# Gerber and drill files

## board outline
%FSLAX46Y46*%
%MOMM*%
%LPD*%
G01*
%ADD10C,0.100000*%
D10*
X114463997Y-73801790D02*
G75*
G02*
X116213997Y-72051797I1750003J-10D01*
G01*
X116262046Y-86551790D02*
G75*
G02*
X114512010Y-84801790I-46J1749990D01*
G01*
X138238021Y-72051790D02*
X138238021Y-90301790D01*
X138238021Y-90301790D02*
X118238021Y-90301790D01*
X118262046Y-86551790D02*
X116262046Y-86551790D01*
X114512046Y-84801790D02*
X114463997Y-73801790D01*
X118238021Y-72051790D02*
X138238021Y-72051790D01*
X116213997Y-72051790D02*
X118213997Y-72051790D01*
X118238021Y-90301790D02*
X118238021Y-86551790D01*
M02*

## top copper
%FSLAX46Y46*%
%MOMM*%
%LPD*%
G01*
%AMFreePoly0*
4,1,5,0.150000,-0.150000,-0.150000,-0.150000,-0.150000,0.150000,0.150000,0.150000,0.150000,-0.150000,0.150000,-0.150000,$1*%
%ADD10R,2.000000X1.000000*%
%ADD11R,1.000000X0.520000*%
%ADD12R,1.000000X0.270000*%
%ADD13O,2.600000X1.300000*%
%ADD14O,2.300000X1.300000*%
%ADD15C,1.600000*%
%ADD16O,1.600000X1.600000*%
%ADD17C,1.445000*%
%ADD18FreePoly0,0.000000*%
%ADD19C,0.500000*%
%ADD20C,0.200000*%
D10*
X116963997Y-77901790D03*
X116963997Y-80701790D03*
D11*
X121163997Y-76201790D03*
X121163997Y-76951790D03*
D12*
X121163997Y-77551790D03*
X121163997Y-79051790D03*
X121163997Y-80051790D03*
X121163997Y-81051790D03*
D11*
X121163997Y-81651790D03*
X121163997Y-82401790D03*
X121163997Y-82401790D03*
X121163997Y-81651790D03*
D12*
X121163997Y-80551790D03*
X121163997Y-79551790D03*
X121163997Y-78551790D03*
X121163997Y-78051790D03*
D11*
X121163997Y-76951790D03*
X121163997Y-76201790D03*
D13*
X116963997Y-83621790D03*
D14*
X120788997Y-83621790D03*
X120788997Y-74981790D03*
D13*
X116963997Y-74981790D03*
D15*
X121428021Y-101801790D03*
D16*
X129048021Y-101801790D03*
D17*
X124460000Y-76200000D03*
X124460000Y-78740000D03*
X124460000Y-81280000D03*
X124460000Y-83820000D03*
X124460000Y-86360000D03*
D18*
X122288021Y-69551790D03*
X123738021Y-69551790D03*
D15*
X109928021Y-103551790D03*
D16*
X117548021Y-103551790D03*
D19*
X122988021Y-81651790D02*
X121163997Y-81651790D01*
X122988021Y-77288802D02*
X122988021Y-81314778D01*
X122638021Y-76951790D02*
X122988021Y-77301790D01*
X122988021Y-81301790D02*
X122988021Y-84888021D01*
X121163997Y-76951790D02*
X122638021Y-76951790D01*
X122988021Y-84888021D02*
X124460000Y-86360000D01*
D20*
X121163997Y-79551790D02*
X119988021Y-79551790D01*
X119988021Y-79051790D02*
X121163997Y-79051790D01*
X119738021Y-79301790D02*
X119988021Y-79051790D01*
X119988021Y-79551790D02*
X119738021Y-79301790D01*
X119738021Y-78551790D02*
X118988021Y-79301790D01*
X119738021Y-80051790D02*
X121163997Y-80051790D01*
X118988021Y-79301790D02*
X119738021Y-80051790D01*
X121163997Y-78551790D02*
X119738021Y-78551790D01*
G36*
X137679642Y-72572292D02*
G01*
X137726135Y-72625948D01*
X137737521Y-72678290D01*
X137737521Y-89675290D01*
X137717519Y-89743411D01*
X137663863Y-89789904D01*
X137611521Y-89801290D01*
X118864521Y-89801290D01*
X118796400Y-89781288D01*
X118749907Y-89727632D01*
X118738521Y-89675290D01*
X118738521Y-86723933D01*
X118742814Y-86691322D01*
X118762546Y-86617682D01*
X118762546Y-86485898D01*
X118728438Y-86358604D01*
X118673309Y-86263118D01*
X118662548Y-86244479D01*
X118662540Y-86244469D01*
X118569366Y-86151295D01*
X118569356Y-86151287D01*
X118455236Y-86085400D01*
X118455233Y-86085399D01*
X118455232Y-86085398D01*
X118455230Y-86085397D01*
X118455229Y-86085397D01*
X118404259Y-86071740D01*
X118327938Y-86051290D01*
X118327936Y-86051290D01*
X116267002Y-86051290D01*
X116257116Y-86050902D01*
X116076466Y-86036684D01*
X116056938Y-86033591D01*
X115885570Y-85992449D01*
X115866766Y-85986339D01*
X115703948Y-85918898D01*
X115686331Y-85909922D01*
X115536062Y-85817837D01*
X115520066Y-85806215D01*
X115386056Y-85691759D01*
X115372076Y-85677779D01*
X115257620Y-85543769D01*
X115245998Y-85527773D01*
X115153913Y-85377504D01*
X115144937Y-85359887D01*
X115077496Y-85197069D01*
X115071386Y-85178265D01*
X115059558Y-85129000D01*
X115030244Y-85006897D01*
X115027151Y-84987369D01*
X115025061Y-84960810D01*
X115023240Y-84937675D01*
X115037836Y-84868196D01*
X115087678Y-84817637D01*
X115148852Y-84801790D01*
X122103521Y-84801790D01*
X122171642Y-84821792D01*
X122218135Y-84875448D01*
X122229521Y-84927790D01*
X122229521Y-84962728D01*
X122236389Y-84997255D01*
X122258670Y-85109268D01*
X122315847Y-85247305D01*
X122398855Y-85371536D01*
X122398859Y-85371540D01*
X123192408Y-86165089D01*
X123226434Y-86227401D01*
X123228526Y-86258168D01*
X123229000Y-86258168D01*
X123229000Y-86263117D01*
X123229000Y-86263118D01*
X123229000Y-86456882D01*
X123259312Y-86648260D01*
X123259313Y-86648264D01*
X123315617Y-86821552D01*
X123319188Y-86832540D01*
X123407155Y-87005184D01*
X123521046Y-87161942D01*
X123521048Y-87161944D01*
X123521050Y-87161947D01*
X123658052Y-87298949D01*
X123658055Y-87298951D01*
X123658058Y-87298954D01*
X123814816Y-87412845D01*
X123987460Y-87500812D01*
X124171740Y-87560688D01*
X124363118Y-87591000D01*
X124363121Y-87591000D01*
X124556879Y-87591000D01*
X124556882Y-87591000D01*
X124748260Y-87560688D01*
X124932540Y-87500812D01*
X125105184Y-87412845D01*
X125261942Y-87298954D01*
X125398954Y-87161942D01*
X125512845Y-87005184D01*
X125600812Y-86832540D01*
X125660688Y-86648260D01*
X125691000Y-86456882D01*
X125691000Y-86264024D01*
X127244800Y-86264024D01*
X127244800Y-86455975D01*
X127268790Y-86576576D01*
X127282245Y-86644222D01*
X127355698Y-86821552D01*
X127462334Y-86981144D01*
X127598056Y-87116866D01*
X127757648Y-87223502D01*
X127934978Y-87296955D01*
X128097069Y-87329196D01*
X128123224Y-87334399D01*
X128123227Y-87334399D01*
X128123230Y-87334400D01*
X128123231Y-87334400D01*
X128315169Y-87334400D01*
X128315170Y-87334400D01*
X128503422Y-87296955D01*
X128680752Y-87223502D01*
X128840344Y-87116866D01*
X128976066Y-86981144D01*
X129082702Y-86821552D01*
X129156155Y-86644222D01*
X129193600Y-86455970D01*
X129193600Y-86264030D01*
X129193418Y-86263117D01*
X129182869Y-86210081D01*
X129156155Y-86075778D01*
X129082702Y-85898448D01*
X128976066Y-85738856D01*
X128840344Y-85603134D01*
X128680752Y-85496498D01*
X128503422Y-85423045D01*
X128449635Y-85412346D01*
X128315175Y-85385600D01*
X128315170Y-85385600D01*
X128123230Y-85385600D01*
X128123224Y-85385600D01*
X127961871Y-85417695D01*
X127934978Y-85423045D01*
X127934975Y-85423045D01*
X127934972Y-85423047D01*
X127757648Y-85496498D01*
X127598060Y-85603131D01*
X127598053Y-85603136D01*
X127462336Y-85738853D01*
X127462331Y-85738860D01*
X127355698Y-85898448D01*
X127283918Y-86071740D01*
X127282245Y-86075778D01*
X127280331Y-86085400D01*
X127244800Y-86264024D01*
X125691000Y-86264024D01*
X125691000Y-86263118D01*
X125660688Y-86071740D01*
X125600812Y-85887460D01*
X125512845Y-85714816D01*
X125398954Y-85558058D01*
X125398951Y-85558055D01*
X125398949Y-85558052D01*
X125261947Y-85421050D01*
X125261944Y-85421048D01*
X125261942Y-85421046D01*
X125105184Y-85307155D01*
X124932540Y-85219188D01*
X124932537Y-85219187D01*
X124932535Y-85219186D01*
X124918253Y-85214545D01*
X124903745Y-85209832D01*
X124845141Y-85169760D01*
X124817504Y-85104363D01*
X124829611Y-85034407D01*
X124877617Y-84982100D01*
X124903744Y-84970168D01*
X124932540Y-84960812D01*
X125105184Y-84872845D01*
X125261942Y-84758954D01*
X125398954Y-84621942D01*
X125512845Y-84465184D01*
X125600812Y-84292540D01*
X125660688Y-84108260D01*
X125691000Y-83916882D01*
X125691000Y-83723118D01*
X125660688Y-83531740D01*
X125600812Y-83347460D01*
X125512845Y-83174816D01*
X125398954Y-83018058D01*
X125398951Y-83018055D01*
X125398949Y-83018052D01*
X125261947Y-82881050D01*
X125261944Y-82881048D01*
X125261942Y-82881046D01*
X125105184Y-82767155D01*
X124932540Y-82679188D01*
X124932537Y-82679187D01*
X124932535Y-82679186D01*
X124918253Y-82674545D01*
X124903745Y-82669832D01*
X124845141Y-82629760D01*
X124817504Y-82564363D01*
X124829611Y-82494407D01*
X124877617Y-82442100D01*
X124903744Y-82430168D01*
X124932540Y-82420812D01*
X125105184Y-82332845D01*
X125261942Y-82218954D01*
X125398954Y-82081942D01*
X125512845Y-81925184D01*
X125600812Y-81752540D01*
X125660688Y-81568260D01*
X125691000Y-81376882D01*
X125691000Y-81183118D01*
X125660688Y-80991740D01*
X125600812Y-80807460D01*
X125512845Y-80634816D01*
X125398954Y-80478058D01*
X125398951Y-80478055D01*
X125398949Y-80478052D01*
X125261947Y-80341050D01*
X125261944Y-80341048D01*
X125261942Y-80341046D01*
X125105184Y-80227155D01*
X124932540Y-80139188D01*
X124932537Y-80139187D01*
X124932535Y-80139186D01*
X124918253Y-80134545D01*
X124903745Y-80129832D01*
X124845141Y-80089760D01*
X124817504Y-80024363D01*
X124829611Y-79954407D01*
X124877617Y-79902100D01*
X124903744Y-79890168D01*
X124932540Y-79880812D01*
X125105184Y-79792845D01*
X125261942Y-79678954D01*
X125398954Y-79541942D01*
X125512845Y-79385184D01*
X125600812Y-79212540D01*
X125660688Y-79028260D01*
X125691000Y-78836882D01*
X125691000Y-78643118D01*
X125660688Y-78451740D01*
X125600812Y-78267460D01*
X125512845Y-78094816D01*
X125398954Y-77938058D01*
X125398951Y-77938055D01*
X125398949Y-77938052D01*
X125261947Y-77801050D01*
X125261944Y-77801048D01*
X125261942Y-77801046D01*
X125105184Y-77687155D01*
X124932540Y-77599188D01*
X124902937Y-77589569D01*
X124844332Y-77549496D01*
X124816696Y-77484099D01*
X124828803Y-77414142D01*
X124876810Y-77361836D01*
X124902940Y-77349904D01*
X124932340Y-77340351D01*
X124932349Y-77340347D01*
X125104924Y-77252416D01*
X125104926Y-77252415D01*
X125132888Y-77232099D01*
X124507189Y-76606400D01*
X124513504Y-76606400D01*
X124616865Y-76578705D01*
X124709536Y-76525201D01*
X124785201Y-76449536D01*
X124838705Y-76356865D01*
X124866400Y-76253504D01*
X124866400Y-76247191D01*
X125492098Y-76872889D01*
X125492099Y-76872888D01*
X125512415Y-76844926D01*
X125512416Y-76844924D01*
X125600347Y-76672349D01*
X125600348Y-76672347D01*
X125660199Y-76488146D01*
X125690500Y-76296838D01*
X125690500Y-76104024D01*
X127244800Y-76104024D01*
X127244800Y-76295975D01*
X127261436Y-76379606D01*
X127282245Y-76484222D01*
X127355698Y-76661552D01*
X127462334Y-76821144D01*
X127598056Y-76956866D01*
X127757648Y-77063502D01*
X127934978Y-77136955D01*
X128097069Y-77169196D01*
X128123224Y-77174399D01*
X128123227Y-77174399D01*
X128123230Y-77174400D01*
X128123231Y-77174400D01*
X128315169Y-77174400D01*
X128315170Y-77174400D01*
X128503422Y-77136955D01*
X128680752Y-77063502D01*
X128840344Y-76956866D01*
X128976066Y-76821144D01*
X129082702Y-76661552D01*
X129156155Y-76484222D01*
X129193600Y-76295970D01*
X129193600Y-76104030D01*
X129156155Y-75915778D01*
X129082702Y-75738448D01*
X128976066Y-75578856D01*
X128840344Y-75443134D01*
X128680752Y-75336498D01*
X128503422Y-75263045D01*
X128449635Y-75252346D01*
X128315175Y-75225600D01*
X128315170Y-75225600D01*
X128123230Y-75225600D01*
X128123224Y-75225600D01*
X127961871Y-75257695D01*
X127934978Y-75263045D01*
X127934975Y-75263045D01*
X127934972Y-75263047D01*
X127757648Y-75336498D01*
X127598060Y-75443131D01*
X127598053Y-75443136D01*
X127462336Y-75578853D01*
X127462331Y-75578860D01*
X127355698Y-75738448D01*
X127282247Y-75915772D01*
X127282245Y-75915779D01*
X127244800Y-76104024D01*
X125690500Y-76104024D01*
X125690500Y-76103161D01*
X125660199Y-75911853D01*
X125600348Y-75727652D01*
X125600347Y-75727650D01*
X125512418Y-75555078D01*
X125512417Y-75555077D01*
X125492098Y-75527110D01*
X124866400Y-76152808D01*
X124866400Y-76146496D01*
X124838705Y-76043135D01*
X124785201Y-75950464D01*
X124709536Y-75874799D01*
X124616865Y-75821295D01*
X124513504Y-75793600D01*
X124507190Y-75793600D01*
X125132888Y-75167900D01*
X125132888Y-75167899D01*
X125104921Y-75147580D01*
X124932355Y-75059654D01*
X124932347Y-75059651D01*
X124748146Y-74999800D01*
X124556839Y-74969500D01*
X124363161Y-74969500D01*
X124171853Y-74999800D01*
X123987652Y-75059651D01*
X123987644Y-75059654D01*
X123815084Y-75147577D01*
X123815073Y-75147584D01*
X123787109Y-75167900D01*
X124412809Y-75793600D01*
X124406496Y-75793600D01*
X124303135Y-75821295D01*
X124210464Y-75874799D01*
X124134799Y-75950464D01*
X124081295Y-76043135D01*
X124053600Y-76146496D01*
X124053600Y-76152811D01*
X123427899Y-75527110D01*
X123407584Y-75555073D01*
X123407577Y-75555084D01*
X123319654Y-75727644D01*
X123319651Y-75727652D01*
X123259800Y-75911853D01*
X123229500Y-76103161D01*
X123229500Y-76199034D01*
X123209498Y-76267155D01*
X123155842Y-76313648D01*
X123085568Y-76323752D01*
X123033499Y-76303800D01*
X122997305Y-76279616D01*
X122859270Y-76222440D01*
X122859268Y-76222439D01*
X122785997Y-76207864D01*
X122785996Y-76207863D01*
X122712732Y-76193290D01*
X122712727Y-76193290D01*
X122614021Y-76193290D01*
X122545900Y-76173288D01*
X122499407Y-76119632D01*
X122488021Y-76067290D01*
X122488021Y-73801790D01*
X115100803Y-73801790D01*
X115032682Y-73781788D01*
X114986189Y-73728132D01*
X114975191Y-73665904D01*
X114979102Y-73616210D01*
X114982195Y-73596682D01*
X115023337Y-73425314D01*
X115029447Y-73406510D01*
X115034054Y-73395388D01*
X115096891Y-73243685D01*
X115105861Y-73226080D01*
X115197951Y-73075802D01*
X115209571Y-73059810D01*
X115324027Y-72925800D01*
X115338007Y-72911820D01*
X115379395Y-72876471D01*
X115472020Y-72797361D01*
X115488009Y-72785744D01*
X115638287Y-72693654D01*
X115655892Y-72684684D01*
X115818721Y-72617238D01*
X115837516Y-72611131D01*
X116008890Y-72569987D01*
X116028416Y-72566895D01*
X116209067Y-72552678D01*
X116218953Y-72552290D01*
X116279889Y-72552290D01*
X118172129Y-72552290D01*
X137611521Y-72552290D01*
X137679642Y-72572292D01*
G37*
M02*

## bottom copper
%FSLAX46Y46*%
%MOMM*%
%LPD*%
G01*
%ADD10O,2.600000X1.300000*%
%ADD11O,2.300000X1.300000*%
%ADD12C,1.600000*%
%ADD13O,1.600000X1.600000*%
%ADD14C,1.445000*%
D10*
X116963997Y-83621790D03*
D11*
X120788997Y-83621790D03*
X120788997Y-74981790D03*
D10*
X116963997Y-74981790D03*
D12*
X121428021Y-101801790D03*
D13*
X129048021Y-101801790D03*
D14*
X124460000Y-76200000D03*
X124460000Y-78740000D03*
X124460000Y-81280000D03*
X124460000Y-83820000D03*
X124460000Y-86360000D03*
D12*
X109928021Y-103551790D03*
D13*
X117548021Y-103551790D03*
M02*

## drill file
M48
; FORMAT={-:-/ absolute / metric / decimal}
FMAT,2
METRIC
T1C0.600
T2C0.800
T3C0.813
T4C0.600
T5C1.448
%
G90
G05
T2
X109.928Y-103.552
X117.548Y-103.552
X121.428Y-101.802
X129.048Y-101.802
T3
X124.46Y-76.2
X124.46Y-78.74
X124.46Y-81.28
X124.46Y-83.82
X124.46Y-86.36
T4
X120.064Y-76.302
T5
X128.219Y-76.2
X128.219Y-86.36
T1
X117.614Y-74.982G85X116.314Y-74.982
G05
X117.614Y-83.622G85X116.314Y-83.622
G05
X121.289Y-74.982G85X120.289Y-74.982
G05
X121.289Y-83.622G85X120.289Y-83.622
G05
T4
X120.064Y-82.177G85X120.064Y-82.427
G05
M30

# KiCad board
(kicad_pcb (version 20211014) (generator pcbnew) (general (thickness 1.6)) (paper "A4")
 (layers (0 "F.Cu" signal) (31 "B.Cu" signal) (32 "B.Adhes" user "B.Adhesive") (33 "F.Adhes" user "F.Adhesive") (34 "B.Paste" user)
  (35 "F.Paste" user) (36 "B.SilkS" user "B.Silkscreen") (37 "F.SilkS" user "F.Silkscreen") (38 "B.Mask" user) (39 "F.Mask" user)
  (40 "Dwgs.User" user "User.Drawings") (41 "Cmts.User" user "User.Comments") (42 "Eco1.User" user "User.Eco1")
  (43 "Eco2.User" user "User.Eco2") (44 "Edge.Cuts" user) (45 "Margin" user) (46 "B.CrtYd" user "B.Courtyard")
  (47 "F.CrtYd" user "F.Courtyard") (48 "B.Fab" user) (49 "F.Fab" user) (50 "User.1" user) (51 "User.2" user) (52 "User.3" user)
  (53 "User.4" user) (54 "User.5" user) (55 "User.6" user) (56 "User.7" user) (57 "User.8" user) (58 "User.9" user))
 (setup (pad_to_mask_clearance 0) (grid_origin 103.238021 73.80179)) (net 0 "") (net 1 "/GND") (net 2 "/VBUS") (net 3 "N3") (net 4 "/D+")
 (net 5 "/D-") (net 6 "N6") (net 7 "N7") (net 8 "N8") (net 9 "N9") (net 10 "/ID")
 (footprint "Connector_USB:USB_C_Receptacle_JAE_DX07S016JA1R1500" (layer "F.Cu") (at 118.113997 79.30179 -90)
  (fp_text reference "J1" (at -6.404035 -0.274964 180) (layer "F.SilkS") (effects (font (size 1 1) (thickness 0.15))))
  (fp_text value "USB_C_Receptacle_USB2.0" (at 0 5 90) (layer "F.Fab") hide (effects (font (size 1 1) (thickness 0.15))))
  (pad "" smd rect (at -1.4 1.15 270) (size 1 2) (layers "F.Cu" "F.Paste" "F.Mask"))
  (pad "" np_thru_hole circle (at -3 -1.95 270) (size 0.6 0.6) (drill 0.6) (layers F&B.Cu *.Mask))
  (pad "" np_thru_hole oval (at 3 -1.95 270) (size 0.85 0.6) (drill oval 0.85 0.6) (layers F&B.Cu *.Mask))
  (pad "" smd rect (at 1.4 1.15 270) (size 1 2) (layers "F.Cu" "F.Paste" "F.Mask"))
  (pad "A1" smd rect (at -3.1 -3.05 270) (size 0.52 1) (layers "F.Cu" "F.Paste" "F.Mask") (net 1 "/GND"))
  (pad "A4" smd rect (at -2.35 -3.05 270) (size 0.52 1) (layers "F.Cu" "F.Paste" "F.Mask") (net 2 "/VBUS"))
  (pad "A5" smd rect (at -1.75 -3.05 270) (size 0.27 1) (layers "F.Cu" "F.Paste" "F.Mask") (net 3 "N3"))
  (pad "A6" smd rect (at -0.25 -3.05 270) (size 0.27 1) (layers "F.Cu" "F.Paste" "F.Mask") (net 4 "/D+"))
  (pad "A7" smd rect (at 0.75 -3.05 270) (size 0.27 1) (layers "F.Cu" "F.Paste" "F.Mask") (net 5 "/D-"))
  (pad "A8" smd rect (at 1.75 -3.05 270) (size 0.27 1) (layers "F.Cu" "F.Paste" "F.Mask") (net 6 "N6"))
  (pad "A9" smd rect (at 2.35 -3.05 270) (size 0.52 1) (layers "F.Cu" "F.Paste" "F.Mask") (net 2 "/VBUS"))
  (pad "A12" smd rect (at 3.1 -3.05 270) (size 0.52 1) (layers "F.Cu" "F.Paste" "F.Mask") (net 1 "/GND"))
  (pad "B1" smd rect (at 3.1 -3.05 270) (size 0.52 1) (layers "F.Cu" "F.Paste" "F.Mask") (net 1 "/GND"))
  (pad "B4" smd rect (at 2.35 -3.05 270) (size 0.52 1) (layers "F.Cu" "F.Paste" "F.Mask") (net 2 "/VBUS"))
  (pad "B5" smd rect (at 1.25 -3.05 270) (size 0.27 1) (layers "F.Cu" "F.Paste" "F.Mask") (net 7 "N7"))
  (pad "B6" smd rect (at 0.25 -3.05 270) (size 0.27 1) (layers "F.Cu" "F.Paste" "F.Mask") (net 4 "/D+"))
  (pad "B7" smd rect (at -0.75 -3.05 270) (size 0.27 1) (layers "F.Cu" "F.Paste" "F.Mask") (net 5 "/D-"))
  (pad "B8" smd rect (at -1.25 -3.05 270) (size 0.27 1) (layers "F.Cu" "F.Paste" "F.Mask") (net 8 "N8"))
  (pad "B9" smd rect (at -2.35 -3.05 270) (size 0.52 1) (layers "F.Cu" "F.Paste" "F.Mask") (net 2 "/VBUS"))
  (pad "B12" smd rect (at -3.1 -3.05 270) (size 0.52 1) (layers "F.Cu" "F.Paste" "F.Mask") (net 1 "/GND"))
  (pad "S1" thru_hole oval (at 4.32 1.15 270) (size 1.3 2.6) (drill oval 0.6 1.9) (layers *.Cu *.Mask) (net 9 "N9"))
  (pad "S1" thru_hole oval (at 4.32 -2.675 270) (size 1.3 2.3) (drill oval 0.6 1.6) (layers *.Cu *.Mask) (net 9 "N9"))
  (pad "S1" thru_hole oval (at -4.32 -2.675 270) (size 1.3 2.3) (drill oval 0.6 1.6) (layers *.Cu *.Mask) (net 9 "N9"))
  (pad "S1" thru_hole oval (at -4.32 1.15 270) (size 1.3 2.6) (drill oval 0.6 1.9) (layers *.Cu *.Mask) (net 9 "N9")))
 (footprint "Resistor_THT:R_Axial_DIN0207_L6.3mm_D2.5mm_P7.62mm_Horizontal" (layer "F.Cu") (at 121.428021 101.80179)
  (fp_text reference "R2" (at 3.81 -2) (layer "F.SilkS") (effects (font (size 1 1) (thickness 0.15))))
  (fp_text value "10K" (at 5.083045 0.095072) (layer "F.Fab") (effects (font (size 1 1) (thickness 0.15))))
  (pad "1" thru_hole circle (at 0 0) (size 1.6 1.6) (drill 0.8) (layers *.Cu *.Mask) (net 1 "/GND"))
  (pad "2" thru_hole oval (at 7.62 0) (size 1.6 1.6) (drill 0.8) (layers *.Cu *.Mask) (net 3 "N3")))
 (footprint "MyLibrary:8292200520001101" (layer "F.Cu") (at 124.46 76.2)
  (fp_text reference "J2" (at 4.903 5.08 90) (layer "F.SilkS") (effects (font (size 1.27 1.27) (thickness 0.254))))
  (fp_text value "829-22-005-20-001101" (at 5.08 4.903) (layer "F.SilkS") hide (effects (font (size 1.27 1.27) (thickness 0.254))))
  (pad "" np_thru_hole circle (at 3.7592 10.16 90) (size 1.4478 1.4478) (drill 1.4478) (layers F&B.Cu *.Mask))
  (pad "" np_thru_hole circle (at 3.7592 0 90) (size 1.4478 1.4478) (drill 1.4478) (layers F&B.Cu *.Mask))
  (pad "1" thru_hole circle (at 0 0 90) (size 1.445 1.445) (drill 0.8128) (layers *.Cu *.Mask) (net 1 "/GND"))
  (pad "2" thru_hole circle (at 0 2.54 90) (size 1.445 1.445) (drill 0.8128) (layers *.Cu *.Mask) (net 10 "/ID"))
  (pad "3" thru_hole circle (at 0 5.08 90) (size 1.445 1.445) (drill 0.8128) (layers *.Cu *.Mask) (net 4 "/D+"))
  (pad "4" thru_hole circle (at 0 7.62 90) (size 1.445 1.445) (drill 0.8128) (layers *.Cu *.Mask) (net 5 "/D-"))
  (pad "5" thru_hole circle (at 0 10.16 90) (size 1.445 1.445) (drill 0.8128) (layers *.Cu *.Mask) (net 2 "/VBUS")))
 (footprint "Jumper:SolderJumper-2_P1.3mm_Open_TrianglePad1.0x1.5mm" (layer "F.Cu") (at 123.013021 69.55179)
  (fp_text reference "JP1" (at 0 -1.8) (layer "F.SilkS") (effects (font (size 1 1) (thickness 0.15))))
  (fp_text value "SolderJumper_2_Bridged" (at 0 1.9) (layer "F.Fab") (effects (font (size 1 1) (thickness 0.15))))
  (pad "1" smd custom (at -0.725 0) (size 0.3 0.3) (layers "F.Cu" "F.Mask") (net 1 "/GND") (zone_connect 2)
   (options (clearance outline) (anchor rect)) (primitives))
  (pad "2" smd custom (at 0.725 0) (size 0.3 0.3) (layers "F.Cu" "F.Mask") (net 10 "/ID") (zone_connect 2)
   (options (clearance outline) (anchor rect)) (primitives)))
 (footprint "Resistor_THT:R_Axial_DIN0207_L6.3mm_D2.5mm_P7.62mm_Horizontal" (layer "F.Cu") (at 109.928021 103.55179)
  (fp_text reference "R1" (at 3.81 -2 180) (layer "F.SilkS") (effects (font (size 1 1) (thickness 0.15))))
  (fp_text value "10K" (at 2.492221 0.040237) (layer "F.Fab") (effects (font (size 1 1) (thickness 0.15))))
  (pad "1" thru_hole circle (at 0 0) (size 1.6 1.6) (drill 0.8) (layers *.Cu *.Mask) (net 1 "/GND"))
  (pad "2" thru_hole oval (at 7.62 0) (size 1.6 1.6) (drill 0.8) (layers *.Cu *.Mask) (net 7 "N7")))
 (gr_arc (start 114.463997 73.80179) (mid 114.97656 72.564353) (end 116.213997 72.05179) (layer "Edge.Cuts") (width 0.1))
 (gr_arc (start 116.262046 86.55179) (mid 115.024609 86.039227) (end 114.512046 84.80179) (layer "Edge.Cuts") (width 0.1))
 (gr_line (start 138.238021 72.05179) (end 138.238021 90.30179) (layer "Edge.Cuts") (width 0.1))
 (gr_line (start 138.238021 90.30179) (end 118.238021 90.30179) (layer "Edge.Cuts") (width 0.1))
 (gr_line (start 118.262046 86.55179) (end 116.262046 86.55179) (layer "Edge.Cuts") (width 0.1))
 (gr_line (start 114.512046 84.80179) (end 114.463997 73.80179) (layer "Edge.Cuts") (width 0.1))
 (gr_line (start 118.238021 72.05179) (end 138.238021 72.05179) (layer "Edge.Cuts") (width 0.1))
 (gr_line (start 116.213997 72.05179) (end 118.213997 72.05179) (layer "Edge.Cuts") (width 0.1))
 (gr_line (start 118.238021 90.30179) (end 118.238021 86.55179) (layer "Edge.Cuts") (width 0.1))
 (segment (start 122.988021 81.65179) (end 121.163997 81.65179) (width 0.5) (layer "F.Cu") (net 2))
 (segment (start 122.988021 77.288802) (end 122.988021 81.314778) (width 0.5) (layer "F.Cu") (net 2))
 (segment (start 122.638021 76.95179) (end 122.988021 77.30179) (width 0.5) (layer "F.Cu") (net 2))
 (segment (start 122.988021 81.30179) (end 122.988021 84.888021) (width 0.5) (layer "F.Cu") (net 2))
 (segment (start 121.163997 76.95179) (end 122.638021 76.95179) (width 0.5) (layer "F.Cu") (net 2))
 (segment (start 122.988021 84.888021) (end 124.46 86.36) (width 0.5) (layer "F.Cu") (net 2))
 (segment (start 121.163997 79.55179) (end 119.988021 79.55179) (width 0.2) (layer "F.Cu") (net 4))
 (segment (start 119.988021 79.05179) (end 121.163997 79.05179) (width 0.2) (layer "F.Cu") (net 4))
 (segment (start 119.738021 79.30179) (end 119.988021 79.05179) (width 0.2) (layer "F.Cu") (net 4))
 (segment (start 119.988021 79.55179) (end 119.738021 79.30179) (width 0.2) (layer "F.Cu") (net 4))
 (segment (start 119.738021 78.55179) (end 118.988021 79.30179) (width 0.2) (layer "F.Cu") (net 5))
 (segment (start 119.738021 80.05179) (end 121.163997 80.05179) (width 0.2) (layer "F.Cu") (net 5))
 (segment (start 118.988021 79.30179) (end 119.738021 80.05179) (width 0.2) (layer "F.Cu") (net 5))
 (segment (start 121.163997 78.55179) (end 119.738021 78.55179) (width 0.2) (layer "F.Cu") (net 5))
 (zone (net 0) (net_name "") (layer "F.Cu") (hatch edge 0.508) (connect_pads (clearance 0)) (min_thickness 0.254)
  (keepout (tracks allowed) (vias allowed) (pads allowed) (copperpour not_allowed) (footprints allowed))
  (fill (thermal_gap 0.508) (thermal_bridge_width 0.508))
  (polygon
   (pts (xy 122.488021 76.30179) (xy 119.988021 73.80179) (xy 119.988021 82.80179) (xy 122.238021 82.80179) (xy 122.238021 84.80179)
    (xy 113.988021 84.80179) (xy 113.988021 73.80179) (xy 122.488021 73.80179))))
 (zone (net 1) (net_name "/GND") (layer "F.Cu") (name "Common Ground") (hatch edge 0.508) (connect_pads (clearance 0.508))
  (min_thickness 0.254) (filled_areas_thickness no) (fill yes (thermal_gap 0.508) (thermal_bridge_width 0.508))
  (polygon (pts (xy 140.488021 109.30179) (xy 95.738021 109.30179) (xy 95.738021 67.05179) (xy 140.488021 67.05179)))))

